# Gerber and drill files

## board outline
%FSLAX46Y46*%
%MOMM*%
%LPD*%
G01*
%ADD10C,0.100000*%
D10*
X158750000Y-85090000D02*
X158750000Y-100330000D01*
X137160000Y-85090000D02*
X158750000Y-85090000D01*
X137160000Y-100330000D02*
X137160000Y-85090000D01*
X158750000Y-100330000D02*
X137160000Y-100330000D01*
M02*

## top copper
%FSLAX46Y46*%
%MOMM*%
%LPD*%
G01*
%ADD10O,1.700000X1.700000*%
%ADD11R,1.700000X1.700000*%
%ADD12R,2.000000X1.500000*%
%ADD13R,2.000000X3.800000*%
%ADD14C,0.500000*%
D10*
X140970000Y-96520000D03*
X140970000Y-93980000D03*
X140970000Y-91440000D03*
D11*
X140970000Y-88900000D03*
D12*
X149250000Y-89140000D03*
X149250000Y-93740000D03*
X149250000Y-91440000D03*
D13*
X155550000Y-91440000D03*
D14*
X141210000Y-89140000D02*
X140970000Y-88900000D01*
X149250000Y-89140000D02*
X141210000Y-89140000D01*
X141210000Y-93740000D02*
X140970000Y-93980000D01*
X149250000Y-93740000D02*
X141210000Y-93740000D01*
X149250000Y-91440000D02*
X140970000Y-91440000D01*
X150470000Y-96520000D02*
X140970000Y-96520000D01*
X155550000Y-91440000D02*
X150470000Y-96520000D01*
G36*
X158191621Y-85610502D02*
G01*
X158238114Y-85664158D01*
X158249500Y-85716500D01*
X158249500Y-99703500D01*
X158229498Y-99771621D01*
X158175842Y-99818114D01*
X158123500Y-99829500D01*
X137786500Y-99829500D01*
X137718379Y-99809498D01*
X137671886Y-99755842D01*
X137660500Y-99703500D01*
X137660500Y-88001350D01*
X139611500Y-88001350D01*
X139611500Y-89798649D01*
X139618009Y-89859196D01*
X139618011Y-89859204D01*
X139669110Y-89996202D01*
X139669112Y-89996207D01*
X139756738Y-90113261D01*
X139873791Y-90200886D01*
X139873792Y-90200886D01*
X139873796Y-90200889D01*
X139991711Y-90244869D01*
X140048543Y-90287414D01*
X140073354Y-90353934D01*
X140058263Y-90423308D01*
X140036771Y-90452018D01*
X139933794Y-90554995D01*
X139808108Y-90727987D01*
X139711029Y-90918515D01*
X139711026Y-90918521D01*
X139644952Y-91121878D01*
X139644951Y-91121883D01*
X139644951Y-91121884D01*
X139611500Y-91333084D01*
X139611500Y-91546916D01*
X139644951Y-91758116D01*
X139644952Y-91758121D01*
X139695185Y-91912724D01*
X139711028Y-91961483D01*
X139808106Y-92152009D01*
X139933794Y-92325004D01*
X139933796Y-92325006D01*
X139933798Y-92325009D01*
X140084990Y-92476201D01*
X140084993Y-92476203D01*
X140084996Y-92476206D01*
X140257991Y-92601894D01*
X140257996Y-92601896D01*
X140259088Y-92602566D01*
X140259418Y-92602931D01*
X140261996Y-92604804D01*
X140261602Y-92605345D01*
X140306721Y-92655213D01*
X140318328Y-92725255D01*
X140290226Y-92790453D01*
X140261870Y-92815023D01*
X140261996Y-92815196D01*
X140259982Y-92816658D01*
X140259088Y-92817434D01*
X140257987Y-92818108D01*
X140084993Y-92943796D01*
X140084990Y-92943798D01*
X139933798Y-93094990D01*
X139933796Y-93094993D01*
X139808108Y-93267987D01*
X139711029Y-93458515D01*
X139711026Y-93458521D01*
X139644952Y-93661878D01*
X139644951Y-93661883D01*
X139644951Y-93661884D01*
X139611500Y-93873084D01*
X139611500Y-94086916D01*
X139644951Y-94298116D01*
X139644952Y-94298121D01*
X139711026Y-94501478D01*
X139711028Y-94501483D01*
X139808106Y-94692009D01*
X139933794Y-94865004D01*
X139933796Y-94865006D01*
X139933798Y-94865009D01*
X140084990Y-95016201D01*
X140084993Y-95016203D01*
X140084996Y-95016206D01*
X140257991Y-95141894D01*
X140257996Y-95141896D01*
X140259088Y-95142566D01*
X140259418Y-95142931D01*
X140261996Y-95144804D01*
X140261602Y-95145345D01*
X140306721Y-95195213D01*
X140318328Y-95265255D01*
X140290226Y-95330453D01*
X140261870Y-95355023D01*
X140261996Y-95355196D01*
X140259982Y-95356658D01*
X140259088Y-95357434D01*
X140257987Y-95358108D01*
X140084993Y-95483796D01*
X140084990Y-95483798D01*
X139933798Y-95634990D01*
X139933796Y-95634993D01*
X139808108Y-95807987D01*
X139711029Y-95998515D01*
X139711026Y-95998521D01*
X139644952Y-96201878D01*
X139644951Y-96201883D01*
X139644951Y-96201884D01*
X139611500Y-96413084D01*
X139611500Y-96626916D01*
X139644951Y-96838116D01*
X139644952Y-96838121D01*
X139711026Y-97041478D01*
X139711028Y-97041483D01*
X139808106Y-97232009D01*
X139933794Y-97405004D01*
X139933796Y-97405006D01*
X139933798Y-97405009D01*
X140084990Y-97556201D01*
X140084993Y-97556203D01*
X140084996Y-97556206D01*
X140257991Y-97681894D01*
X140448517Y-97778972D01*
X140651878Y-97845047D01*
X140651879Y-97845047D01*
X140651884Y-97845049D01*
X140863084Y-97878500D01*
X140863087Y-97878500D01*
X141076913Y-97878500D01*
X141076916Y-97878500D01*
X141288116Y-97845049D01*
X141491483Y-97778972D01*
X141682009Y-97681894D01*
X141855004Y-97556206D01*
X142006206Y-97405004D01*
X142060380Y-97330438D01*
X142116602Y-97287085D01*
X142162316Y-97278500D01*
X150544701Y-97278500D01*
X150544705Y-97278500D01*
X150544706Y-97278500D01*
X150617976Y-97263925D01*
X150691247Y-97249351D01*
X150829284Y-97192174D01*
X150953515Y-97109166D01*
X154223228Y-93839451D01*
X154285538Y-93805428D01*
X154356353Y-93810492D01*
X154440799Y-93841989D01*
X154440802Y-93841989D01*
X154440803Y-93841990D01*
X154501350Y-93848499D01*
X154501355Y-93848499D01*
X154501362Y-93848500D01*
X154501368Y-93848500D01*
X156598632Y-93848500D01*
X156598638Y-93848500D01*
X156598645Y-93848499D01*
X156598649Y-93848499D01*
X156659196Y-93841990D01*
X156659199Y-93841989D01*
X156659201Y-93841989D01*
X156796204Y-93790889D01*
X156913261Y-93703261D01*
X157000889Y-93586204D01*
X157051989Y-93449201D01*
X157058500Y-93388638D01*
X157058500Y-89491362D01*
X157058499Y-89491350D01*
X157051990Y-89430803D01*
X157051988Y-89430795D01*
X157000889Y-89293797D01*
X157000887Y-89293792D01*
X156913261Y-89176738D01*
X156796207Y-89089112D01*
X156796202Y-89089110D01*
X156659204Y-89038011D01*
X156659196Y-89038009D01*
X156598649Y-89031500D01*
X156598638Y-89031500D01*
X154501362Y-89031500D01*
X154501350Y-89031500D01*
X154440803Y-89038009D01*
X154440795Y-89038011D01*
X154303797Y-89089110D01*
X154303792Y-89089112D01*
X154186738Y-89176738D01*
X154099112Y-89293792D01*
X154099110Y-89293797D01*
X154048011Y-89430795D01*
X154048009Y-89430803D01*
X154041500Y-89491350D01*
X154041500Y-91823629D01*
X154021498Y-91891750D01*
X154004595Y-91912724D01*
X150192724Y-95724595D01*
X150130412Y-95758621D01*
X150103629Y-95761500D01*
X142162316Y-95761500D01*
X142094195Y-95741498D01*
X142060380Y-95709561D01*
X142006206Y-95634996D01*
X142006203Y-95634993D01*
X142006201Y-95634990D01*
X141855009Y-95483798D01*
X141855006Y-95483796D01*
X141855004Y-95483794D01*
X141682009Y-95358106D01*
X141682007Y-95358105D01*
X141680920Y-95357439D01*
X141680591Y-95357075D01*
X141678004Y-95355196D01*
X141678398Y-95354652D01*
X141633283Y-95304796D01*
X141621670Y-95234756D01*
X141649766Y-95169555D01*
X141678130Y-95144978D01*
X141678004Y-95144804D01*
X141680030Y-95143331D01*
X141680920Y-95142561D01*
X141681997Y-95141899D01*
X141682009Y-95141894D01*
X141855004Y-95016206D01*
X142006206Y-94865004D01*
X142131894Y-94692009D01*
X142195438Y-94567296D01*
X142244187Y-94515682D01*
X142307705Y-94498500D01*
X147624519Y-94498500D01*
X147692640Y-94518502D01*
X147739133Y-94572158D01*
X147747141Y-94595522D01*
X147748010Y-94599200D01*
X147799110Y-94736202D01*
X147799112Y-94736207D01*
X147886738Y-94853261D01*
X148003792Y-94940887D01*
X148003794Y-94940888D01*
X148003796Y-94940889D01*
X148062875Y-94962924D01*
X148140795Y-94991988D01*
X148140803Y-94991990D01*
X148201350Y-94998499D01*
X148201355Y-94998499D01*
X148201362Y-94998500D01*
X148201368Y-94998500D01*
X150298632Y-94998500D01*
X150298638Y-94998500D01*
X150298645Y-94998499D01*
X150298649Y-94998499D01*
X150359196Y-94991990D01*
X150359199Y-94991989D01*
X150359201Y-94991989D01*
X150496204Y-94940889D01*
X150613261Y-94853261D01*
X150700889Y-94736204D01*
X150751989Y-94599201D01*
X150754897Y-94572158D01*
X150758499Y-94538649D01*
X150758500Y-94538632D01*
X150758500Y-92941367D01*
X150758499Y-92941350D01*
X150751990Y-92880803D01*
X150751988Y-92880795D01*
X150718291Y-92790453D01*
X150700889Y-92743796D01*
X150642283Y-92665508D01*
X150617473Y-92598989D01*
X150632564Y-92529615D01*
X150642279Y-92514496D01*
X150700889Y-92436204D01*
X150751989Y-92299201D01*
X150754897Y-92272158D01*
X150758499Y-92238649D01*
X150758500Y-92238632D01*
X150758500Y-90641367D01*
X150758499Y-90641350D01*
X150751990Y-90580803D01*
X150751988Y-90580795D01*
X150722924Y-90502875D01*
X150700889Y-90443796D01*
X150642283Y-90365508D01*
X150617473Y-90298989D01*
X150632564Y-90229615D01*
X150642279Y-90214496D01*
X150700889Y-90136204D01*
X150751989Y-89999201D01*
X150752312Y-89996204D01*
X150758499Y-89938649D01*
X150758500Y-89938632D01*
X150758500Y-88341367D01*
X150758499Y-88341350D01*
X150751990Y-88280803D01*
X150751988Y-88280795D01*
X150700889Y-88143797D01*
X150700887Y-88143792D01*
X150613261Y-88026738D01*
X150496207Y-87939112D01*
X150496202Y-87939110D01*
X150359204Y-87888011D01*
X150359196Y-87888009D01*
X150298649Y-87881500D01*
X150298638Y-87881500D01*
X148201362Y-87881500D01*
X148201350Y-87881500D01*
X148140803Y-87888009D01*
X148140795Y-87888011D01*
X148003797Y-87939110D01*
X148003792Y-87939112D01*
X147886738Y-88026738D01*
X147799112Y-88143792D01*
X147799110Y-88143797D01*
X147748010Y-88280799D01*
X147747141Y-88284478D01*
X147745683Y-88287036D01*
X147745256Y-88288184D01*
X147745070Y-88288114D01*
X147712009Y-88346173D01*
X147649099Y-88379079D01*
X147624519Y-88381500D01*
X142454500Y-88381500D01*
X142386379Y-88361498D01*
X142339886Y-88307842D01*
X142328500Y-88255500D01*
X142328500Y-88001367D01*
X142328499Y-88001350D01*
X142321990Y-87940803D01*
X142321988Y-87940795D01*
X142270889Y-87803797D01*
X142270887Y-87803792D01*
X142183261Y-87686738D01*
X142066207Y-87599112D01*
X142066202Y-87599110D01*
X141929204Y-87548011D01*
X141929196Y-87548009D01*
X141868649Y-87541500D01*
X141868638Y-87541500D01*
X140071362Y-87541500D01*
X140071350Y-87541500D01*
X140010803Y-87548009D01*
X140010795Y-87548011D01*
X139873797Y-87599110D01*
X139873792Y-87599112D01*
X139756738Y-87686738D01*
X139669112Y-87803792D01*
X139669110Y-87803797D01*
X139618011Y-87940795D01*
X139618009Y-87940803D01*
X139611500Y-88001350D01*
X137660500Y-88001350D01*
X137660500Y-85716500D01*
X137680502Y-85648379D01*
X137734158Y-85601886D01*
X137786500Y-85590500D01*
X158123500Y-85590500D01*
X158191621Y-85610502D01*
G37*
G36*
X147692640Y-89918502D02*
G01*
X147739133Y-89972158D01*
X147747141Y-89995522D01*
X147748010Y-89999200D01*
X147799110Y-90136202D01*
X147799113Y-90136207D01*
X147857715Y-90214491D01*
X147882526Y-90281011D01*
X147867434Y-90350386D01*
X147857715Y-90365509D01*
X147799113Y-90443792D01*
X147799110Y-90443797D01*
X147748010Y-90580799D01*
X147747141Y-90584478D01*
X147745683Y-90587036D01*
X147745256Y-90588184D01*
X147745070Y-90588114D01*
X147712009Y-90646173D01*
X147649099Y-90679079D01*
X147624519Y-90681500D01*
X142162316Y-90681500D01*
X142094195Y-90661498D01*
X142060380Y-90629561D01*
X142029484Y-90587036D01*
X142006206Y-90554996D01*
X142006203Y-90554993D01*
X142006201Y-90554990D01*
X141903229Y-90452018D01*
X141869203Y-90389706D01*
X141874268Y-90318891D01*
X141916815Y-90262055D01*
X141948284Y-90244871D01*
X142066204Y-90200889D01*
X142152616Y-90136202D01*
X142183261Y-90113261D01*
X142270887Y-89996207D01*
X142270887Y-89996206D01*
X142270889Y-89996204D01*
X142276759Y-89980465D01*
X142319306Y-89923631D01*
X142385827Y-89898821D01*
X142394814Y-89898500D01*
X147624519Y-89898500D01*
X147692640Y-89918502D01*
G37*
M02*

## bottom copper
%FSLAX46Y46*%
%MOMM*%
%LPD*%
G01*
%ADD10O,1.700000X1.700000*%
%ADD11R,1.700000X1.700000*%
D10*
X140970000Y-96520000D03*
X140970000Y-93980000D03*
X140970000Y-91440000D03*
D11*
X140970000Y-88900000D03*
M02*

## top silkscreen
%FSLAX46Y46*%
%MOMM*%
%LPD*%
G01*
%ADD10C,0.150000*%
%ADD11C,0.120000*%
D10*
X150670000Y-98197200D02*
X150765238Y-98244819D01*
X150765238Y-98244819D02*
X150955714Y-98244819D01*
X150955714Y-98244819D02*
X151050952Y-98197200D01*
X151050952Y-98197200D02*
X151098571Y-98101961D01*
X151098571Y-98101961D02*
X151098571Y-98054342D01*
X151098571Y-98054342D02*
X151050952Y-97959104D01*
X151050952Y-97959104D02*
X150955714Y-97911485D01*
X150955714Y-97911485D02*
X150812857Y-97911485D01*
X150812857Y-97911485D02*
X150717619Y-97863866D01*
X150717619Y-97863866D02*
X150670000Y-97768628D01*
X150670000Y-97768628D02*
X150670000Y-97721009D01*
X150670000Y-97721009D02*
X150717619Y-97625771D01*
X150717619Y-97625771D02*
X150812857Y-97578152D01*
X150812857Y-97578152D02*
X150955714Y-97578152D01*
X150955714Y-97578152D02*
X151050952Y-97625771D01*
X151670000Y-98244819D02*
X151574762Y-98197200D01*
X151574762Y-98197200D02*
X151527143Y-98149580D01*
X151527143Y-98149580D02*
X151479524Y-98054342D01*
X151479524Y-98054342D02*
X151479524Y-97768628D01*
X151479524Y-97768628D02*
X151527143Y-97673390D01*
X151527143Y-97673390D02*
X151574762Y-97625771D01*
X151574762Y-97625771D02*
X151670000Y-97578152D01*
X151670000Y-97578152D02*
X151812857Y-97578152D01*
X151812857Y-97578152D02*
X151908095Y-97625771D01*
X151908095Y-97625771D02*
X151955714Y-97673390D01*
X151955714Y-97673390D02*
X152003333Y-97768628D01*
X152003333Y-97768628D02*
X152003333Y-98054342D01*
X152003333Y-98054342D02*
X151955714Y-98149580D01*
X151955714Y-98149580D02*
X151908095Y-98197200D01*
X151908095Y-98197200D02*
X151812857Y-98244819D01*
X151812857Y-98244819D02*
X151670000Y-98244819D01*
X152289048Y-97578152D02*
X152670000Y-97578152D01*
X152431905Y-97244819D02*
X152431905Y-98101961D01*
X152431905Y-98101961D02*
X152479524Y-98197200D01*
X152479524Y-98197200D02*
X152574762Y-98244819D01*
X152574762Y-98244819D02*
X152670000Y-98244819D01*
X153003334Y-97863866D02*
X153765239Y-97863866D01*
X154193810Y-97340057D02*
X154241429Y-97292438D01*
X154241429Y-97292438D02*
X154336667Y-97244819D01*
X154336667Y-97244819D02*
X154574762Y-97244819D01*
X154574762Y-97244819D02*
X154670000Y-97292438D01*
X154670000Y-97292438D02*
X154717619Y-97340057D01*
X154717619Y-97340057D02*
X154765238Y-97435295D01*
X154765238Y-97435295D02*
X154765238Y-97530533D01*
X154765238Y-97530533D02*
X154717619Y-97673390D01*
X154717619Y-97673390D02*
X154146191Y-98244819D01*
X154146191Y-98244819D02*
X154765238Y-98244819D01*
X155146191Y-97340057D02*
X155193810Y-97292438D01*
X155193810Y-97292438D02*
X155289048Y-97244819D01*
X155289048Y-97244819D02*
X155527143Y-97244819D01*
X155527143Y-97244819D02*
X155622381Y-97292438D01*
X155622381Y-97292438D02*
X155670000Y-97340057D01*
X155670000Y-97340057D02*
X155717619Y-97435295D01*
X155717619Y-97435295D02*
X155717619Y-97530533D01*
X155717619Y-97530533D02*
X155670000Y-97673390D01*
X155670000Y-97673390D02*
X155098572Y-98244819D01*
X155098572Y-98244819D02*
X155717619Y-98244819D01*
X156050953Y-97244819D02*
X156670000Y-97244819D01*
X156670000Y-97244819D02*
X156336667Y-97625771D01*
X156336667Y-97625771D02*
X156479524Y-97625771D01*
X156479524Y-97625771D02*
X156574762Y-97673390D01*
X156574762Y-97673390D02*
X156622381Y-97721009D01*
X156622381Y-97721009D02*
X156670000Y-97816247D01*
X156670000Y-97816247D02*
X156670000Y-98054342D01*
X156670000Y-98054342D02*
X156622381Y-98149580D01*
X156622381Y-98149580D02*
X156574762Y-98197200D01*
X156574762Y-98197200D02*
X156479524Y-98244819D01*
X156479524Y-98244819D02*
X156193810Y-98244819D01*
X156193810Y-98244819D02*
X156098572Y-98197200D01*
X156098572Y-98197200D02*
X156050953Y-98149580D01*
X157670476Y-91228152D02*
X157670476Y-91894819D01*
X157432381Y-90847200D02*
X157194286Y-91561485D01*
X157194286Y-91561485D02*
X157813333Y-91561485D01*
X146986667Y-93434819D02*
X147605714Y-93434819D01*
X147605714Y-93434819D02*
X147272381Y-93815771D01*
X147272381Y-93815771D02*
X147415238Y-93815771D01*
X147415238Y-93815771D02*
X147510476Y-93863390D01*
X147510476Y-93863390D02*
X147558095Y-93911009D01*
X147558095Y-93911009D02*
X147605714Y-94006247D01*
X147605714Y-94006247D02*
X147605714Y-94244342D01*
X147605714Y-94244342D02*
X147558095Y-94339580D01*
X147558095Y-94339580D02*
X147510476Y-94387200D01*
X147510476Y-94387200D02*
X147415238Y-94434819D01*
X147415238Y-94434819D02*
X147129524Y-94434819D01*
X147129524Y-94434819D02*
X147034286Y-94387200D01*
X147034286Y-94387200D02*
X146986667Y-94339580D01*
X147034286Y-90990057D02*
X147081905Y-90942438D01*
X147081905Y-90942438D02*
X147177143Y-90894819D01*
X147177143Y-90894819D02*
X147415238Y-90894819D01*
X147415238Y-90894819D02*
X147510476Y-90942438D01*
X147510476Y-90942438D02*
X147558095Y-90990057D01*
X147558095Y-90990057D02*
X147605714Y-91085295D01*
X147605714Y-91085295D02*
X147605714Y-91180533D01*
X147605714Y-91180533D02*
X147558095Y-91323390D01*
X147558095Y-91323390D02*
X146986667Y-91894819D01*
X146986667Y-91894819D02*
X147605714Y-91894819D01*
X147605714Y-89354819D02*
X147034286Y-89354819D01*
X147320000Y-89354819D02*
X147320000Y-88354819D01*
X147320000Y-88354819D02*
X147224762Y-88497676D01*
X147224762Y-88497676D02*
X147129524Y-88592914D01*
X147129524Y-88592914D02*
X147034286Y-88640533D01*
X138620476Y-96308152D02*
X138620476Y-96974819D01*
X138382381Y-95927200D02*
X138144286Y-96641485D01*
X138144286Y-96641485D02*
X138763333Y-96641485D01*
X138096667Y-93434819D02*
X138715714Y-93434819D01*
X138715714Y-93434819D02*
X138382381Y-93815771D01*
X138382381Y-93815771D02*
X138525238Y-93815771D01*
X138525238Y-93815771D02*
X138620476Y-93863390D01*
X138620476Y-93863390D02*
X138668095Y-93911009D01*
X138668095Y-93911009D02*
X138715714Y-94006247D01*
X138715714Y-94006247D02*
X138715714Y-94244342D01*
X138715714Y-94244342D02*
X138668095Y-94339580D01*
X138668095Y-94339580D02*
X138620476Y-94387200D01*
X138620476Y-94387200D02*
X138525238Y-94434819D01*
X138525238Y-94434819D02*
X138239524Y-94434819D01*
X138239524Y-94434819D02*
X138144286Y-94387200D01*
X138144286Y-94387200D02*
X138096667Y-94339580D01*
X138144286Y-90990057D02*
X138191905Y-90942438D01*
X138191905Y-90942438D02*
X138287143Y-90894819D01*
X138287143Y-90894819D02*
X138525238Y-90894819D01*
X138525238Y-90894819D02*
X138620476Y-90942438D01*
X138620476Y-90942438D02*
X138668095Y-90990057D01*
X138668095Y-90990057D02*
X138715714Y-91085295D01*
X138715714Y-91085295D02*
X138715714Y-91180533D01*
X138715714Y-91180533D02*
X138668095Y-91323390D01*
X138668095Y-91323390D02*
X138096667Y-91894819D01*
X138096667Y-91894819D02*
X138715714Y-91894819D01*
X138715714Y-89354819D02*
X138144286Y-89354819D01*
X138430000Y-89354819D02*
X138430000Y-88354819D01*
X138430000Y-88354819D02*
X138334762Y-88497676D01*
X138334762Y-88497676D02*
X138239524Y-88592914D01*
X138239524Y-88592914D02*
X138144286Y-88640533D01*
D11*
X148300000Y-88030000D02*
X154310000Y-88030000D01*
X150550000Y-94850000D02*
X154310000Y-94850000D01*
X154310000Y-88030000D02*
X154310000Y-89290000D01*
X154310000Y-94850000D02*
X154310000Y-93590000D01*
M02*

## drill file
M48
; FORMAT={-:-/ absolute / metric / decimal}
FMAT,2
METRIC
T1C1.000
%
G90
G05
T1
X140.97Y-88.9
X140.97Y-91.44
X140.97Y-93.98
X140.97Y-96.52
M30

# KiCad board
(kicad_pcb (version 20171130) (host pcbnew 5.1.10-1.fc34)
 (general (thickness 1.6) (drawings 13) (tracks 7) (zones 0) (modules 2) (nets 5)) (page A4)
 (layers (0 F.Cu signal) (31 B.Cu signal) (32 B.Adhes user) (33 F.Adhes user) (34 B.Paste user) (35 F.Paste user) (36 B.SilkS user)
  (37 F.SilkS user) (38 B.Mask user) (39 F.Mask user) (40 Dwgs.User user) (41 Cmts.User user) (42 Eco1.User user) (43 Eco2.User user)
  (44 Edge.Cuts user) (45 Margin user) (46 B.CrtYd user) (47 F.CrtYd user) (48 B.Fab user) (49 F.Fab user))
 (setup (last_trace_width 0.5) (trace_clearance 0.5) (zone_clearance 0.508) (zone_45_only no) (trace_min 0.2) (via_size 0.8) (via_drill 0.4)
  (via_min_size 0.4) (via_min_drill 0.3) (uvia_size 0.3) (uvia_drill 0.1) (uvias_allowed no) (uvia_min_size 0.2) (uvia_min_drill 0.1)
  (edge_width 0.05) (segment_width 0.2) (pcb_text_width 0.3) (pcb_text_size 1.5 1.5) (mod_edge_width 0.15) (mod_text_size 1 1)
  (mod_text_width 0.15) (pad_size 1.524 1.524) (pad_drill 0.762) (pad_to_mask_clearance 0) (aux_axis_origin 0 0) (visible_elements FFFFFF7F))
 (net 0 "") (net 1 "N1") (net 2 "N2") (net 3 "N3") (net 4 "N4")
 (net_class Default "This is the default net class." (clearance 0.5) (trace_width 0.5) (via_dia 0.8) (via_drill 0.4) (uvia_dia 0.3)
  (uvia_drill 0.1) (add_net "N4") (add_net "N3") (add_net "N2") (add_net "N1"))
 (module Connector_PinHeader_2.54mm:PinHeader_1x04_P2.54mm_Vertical (layer B.Cu) (at 140.97 88.9 180)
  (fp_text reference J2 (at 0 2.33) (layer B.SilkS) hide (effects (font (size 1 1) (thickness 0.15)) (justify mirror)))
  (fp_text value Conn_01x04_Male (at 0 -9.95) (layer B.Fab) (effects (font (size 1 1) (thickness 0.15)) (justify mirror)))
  (pad 4 thru_hole oval (at 0 -7.62 180) (size 1.7 1.7) (drill 1) (layers *.Cu *.Mask) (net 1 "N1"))
  (pad 3 thru_hole oval (at 0 -5.08 180) (size 1.7 1.7) (drill 1) (layers *.Cu *.Mask) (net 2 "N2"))
  (pad 2 thru_hole oval (at 0 -2.54 180) (size 1.7 1.7) (drill 1) (layers *.Cu *.Mask) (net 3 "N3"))
  (pad 1 thru_hole rect (at 0 0 180) (size 1.7 1.7) (drill 1) (layers *.Cu *.Mask) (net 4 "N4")))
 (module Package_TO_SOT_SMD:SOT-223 (layer F.Cu) (at 152.4 91.44)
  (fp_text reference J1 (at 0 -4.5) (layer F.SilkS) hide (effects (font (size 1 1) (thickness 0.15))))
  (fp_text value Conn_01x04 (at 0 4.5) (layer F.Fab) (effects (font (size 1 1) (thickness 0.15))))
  (fp_line (start -4.1 -3.41) (end 1.91 -3.41) (layer F.SilkS) (width 0.12))
  (fp_line (start -1.85 3.41) (end 1.91 3.41) (layer F.SilkS) (width 0.12))
  (fp_line (start 1.91 -3.41) (end 1.91 -2.15) (layer F.SilkS) (width 0.12))
  (fp_line (start 1.91 3.41) (end 1.91 2.15) (layer F.SilkS) (width 0.12))
  (pad 1 smd rect (at -3.15 -2.3) (size 2 1.5) (layers F.Cu F.Paste F.Mask) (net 4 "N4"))
  (pad 3 smd rect (at -3.15 2.3) (size 2 1.5) (layers F.Cu F.Paste F.Mask) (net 2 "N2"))
  (pad 2 smd rect (at -3.15 0) (size 2 1.5) (layers F.Cu F.Paste F.Mask) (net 3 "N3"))
  (pad 4 smd rect (at 3.15 0) (size 2 3.8) (layers F.Cu F.Paste F.Mask) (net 1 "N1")))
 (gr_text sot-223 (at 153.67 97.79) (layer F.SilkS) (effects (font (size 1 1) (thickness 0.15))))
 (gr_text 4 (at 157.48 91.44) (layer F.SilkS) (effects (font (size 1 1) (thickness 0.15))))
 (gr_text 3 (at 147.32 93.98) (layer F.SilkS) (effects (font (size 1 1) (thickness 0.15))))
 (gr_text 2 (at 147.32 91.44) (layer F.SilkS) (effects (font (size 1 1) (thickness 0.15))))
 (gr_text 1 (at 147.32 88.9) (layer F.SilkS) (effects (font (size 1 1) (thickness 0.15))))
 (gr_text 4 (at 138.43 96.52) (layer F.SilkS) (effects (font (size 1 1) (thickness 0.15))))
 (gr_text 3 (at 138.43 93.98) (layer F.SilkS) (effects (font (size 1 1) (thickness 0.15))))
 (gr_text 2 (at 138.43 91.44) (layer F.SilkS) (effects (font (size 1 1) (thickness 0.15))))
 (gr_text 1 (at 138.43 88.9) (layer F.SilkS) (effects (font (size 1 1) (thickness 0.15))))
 (gr_line (start 158.75 85.09) (end 158.75 100.33) (layer Edge.Cuts) (width 0.1))
 (gr_line (start 137.16 85.09) (end 158.75 85.09) (layer Edge.Cuts) (width 0.1))
 (gr_line (start 137.16 100.33) (end 137.16 85.09) (layer Edge.Cuts) (width 0.1))
 (gr_line (start 158.75 100.33) (end 137.16 100.33) (layer Edge.Cuts) (width 0.1))
 (segment (start 141.21 89.14) (end 140.97 88.9) (width 0.5) (layer F.Cu) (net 4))
 (segment (start 149.25 89.14) (end 141.21 89.14) (width 0.5) (layer F.Cu) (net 4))
 (segment (start 141.21 93.74) (end 140.97 93.98) (width 0.5) (layer F.Cu) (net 2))
 (segment (start 149.25 93.74) (end 141.21 93.74) (width 0.5) (layer F.Cu) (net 2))
 (segment (start 149.25 91.44) (end 140.97 91.44) (width 0.5) (layer F.Cu) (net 3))
 (segment (start 150.47 96.52) (end 140.97 96.52) (width 0.5) (layer F.Cu) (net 1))
 (segment (start 155.55 91.44) (end 150.47 96.52) (width 0.5) (layer F.Cu) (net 1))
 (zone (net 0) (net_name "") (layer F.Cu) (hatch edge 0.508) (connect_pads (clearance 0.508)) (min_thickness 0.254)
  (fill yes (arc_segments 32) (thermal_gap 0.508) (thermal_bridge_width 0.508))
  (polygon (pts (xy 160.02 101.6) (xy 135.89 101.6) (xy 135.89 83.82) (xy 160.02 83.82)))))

